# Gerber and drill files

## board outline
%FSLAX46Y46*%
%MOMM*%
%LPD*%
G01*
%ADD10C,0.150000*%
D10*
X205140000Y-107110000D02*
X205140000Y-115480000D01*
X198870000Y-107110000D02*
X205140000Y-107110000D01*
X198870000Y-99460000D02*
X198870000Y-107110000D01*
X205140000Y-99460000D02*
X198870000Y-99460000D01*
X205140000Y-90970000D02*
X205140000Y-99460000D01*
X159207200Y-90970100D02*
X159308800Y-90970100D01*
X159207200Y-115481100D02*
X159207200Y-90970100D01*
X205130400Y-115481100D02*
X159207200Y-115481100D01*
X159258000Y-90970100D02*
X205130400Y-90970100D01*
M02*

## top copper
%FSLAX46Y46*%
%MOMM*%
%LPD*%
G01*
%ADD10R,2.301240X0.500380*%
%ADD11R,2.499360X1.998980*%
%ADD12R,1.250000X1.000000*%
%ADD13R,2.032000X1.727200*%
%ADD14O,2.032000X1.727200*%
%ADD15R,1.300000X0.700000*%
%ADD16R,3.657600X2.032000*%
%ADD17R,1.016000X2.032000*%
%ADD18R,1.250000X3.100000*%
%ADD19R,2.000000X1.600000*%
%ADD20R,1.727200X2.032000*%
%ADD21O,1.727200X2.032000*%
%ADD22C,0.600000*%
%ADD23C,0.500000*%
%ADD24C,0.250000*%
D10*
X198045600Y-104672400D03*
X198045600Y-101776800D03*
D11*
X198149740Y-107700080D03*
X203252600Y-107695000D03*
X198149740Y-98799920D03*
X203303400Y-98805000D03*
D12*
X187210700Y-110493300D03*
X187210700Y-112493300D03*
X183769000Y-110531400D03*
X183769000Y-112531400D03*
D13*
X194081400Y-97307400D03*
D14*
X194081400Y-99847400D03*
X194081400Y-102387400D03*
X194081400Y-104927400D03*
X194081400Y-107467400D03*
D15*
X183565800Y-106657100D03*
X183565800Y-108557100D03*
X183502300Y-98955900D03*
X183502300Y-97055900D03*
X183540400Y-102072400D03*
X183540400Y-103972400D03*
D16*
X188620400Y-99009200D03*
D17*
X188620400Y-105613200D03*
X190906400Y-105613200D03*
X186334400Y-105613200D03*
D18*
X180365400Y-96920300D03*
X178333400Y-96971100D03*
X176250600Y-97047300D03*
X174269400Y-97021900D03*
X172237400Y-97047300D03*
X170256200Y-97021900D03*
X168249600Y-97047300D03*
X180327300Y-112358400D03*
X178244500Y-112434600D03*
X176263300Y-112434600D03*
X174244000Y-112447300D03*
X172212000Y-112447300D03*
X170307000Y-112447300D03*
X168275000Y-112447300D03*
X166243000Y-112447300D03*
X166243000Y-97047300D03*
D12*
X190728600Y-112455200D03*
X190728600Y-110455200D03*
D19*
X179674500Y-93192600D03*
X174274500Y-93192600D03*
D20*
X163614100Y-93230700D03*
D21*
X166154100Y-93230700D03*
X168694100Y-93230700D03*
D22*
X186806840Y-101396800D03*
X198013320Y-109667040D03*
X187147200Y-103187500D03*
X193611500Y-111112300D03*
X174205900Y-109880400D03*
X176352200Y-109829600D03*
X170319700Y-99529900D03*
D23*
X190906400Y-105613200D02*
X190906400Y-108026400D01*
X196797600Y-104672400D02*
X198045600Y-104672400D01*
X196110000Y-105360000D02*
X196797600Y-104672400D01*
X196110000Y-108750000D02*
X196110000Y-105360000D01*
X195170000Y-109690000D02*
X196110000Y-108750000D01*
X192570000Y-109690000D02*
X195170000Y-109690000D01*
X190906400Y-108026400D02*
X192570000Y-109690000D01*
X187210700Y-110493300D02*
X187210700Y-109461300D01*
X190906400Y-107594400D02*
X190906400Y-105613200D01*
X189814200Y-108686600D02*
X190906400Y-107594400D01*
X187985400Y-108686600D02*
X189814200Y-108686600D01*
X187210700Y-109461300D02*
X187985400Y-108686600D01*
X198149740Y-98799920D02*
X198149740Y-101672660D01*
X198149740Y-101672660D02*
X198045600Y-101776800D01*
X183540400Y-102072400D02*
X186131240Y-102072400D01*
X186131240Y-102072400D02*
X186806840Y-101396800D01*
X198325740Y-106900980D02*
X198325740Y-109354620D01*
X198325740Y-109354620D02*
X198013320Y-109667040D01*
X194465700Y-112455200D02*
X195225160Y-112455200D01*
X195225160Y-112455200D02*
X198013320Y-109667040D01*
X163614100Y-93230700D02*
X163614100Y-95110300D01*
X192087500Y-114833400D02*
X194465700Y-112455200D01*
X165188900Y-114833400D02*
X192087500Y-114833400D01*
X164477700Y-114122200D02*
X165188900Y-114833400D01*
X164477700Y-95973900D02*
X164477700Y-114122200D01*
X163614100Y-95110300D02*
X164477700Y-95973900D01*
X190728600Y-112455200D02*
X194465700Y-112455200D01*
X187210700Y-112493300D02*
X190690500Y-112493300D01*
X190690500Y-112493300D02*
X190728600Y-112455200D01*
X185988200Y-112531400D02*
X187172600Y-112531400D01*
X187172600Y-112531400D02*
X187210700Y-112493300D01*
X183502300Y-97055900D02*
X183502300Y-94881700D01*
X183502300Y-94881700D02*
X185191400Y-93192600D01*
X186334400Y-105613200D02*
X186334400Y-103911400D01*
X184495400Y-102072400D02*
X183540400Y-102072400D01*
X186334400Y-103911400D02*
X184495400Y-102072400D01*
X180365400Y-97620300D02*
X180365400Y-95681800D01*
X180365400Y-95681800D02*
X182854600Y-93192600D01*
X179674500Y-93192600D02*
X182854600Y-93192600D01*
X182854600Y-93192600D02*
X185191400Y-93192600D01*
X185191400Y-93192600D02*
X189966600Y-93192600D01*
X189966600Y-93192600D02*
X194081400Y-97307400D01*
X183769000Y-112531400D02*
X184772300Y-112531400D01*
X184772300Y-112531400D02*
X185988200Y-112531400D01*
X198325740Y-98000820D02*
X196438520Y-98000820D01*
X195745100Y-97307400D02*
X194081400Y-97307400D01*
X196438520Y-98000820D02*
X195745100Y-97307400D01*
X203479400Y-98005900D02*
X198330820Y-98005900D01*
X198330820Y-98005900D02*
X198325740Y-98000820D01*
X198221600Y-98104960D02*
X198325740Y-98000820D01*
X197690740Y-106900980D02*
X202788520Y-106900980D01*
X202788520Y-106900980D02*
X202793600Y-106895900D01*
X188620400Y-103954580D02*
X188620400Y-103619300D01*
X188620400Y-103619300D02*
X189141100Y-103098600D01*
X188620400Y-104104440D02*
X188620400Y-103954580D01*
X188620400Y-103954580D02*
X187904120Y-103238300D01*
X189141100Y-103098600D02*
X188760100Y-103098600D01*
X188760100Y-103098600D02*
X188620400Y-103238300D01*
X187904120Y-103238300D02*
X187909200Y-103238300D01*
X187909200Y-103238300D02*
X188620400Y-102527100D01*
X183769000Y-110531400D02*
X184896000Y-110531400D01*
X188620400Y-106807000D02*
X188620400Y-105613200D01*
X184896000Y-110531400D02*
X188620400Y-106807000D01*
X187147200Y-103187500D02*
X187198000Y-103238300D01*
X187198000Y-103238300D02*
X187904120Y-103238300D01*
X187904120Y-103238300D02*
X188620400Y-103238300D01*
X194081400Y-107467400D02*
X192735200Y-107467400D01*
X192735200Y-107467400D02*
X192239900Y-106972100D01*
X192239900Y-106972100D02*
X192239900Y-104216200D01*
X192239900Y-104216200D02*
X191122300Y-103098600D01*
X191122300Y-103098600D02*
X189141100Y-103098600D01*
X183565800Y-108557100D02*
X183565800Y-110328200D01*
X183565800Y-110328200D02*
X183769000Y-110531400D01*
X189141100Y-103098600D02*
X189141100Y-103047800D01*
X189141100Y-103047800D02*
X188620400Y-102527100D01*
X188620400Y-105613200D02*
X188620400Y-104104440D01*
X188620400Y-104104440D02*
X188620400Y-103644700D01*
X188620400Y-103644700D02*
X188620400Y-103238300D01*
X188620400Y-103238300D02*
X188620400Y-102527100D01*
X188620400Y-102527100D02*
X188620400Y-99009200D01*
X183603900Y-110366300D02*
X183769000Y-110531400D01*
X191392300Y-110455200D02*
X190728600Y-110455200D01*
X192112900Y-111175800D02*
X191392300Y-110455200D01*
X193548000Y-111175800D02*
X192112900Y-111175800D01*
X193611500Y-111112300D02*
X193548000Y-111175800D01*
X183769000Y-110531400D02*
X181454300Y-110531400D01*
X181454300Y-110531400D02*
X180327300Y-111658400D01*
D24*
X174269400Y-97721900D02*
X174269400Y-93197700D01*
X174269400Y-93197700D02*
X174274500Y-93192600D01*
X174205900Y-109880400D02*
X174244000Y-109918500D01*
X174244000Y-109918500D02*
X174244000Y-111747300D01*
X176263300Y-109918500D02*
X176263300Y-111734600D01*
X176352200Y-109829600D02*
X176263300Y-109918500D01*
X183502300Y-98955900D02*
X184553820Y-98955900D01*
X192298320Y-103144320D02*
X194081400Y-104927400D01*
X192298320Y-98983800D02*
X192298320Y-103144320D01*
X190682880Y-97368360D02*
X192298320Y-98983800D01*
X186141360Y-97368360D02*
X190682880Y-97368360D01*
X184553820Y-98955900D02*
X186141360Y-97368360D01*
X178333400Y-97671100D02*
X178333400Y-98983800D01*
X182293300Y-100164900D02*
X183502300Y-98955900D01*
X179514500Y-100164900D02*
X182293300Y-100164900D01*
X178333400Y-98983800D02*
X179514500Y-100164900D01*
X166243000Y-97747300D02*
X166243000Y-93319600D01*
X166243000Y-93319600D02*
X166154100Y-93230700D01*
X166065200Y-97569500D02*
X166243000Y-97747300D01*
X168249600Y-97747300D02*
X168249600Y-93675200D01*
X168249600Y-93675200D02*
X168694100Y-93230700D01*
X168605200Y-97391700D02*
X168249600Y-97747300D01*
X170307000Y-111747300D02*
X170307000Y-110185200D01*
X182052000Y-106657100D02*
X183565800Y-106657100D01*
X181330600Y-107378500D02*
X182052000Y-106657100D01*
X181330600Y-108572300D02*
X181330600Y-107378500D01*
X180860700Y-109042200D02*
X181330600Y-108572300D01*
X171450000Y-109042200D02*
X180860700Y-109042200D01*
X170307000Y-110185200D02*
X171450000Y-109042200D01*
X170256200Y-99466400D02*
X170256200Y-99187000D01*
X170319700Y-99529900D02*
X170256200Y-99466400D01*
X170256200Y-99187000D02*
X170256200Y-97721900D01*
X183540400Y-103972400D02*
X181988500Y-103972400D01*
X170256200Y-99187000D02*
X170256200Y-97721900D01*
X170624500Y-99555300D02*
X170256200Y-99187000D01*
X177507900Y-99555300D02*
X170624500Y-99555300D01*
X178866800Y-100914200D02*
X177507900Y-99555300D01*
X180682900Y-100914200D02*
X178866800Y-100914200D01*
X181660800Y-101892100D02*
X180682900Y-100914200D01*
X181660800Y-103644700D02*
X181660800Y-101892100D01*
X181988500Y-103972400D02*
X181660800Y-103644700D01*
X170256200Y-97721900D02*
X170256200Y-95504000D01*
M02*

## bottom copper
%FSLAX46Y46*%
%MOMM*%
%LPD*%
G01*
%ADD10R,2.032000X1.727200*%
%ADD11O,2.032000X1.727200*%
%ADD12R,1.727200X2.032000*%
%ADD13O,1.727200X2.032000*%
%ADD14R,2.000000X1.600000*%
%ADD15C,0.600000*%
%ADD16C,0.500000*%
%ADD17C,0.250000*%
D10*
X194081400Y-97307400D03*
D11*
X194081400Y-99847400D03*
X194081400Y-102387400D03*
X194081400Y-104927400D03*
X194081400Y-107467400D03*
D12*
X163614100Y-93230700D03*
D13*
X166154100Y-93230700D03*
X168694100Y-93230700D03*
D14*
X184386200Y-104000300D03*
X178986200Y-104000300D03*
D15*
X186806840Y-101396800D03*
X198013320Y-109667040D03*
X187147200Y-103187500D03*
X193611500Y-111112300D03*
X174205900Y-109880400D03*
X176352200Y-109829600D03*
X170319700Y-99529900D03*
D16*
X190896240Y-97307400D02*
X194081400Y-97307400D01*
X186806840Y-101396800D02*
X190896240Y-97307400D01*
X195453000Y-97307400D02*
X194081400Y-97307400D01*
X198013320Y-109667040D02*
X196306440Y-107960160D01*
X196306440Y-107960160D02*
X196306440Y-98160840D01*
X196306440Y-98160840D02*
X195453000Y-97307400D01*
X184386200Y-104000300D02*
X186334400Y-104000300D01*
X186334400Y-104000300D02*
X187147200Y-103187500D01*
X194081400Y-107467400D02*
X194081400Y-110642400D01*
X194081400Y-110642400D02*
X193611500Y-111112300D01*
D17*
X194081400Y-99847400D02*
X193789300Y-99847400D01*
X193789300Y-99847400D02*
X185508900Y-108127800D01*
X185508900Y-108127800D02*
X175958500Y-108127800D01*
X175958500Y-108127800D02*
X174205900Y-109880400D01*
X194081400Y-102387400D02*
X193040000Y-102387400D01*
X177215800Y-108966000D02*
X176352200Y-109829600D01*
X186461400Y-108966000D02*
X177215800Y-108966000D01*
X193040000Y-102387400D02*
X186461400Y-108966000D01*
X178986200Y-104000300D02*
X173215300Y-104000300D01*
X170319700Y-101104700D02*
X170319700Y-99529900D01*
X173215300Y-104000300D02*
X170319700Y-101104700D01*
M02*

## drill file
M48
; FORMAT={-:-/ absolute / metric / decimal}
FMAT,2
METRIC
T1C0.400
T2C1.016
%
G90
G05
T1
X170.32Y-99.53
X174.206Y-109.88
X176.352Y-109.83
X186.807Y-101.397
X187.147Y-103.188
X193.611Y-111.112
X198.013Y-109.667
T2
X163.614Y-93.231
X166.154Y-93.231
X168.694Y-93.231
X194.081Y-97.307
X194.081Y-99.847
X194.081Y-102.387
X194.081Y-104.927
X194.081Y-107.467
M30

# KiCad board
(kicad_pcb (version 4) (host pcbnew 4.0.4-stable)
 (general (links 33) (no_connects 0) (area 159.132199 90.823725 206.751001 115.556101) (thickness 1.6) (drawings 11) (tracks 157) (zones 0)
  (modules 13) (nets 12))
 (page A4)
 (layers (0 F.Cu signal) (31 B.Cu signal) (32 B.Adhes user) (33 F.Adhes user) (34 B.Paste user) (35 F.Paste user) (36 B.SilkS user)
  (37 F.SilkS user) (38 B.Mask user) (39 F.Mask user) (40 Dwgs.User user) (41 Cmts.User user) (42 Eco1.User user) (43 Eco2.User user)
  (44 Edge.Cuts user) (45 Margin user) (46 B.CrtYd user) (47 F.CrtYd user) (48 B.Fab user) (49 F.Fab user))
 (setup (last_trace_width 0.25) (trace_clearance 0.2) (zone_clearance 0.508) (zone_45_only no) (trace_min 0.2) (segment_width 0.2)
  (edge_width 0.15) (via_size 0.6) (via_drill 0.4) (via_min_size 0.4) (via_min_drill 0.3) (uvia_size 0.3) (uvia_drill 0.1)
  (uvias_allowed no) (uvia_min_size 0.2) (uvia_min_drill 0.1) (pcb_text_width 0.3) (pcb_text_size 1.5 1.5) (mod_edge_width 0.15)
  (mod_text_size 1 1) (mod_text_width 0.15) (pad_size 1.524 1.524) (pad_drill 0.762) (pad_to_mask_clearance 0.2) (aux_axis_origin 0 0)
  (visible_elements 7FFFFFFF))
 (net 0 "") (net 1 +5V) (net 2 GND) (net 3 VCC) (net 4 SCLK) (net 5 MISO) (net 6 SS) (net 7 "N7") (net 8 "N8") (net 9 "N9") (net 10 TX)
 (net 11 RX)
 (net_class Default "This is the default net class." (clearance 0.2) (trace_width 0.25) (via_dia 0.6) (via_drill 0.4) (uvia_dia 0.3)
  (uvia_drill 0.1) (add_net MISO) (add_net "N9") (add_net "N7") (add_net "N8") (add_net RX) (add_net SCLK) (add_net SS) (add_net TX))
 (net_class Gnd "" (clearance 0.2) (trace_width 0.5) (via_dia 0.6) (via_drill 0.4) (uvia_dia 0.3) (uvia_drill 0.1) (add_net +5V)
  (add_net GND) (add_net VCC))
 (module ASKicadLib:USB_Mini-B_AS (layer F.Cu) (at 201.5 103.25 180)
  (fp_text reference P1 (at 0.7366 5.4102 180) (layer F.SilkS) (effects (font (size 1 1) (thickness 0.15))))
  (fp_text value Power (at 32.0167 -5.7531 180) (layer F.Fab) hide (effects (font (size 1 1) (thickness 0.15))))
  (pad 1 smd rect (at 3.4544 -1.4224 180) (size 2.30124 0.50038) (layers F.Cu F.Paste F.Mask) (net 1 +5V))
  (pad 5 smd rect (at 3.4544 1.4732 180) (size 2.30124 0.50038) (layers F.Cu F.Paste F.Mask) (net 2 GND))
  (pad 6 smd rect (at 3.35026 -4.45008 180) (size 2.49936 1.99898) (layers F.Cu F.Paste F.Mask) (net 2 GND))
  (pad 6 smd rect (at -1.7526 -4.445 180) (size 2.49936 1.99898) (layers F.Cu F.Paste F.Mask) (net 2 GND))
  (pad 6 smd rect (at 3.35026 4.45008 180) (size 2.49936 1.99898) (layers F.Cu F.Paste F.Mask) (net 2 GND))
  (pad 6 smd rect (at -1.8034 4.445 180) (size 2.49936 1.99898) (layers F.Cu F.Paste F.Mask) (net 2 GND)))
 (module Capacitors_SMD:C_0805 (layer F.Cu) (at 187.2107 111.4933 270)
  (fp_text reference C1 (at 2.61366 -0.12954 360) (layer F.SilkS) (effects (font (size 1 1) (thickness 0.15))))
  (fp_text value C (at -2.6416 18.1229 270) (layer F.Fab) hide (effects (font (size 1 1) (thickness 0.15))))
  (pad 1 smd rect (at -1 0 270) (size 1 1.25) (layers F.Cu F.Paste F.Mask) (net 1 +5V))
  (pad 2 smd rect (at 1 0 270) (size 1 1.25) (layers F.Cu F.Paste F.Mask) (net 2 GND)))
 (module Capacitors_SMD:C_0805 (layer F.Cu) (at 183.769 111.5314 270)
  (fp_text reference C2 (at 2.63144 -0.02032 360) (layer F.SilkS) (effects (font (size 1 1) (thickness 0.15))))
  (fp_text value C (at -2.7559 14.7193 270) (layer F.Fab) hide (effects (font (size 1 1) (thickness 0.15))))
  (pad 1 smd rect (at -1 0 270) (size 1 1.25) (layers F.Cu F.Paste F.Mask) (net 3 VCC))
  (pad 2 smd rect (at 1 0 270) (size 1 1.25) (layers F.Cu F.Paste F.Mask) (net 2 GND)))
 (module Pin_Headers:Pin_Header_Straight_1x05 (layer F.Cu) (at 194.0814 97.3074)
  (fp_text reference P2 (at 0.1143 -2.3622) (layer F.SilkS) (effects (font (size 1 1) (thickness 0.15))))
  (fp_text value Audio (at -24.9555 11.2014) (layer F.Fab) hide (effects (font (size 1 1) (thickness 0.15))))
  (pad 1 thru_hole rect (at 0 0) (size 2.032 1.7272) (drill 1.016) (layers *.Cu *.Mask) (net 2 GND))
  (pad 2 thru_hole oval (at 0 2.54) (size 2.032 1.7272) (drill 1.016) (layers *.Cu *.Mask) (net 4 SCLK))
  (pad 3 thru_hole oval (at 0 5.08) (size 2.032 1.7272) (drill 1.016) (layers *.Cu *.Mask) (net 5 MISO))
  (pad 4 thru_hole oval (at 0 7.62) (size 2.032 1.7272) (drill 1.016) (layers *.Cu *.Mask) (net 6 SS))
  (pad 5 thru_hole oval (at 0 10.16) (size 2.032 1.7272) (drill 1.016) (layers *.Cu *.Mask) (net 3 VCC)))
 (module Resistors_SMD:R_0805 (layer F.Cu) (at 183.5658 107.6071 270)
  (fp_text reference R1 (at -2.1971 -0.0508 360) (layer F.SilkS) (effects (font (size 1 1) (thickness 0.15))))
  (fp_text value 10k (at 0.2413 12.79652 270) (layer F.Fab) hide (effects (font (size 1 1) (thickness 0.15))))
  (pad 1 smd rect (at -0.95 0 270) (size 0.7 1.3) (layers F.Cu F.Paste F.Mask) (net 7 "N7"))
  (pad 2 smd rect (at 0.95 0 270) (size 0.7 1.3) (layers F.Cu F.Paste F.Mask) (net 3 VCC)))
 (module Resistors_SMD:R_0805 (layer F.Cu) (at 183.5023 98.0059 90)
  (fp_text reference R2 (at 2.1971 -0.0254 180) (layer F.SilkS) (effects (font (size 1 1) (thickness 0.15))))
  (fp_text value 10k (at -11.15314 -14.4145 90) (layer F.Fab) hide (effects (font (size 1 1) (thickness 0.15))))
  (pad 1 smd rect (at -0.95 0 90) (size 0.7 1.3) (layers F.Cu F.Paste F.Mask) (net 6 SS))
  (pad 2 smd rect (at 0.95 0 90) (size 0.7 1.3) (layers F.Cu F.Paste F.Mask) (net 2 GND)))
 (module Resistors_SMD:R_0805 (layer F.Cu) (at 183.5404 103.0224 270)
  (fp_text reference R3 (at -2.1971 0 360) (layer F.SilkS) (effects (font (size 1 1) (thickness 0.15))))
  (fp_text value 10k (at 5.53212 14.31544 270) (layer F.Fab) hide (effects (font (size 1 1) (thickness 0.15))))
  (pad 1 smd rect (at -0.95 0 270) (size 0.7 1.3) (layers F.Cu F.Paste F.Mask) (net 2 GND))
  (pad 2 smd rect (at 0.95 0 270) (size 0.7 1.3) (layers F.Cu F.Paste F.Mask) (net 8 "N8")))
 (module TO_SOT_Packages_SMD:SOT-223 (layer F.Cu) (at 188.6204 102.3112)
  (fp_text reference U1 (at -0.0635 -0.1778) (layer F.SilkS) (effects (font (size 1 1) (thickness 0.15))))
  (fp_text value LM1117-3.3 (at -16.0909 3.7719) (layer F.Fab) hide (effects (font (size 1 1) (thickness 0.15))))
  (pad 4 smd rect (at 0 -3.302) (size 3.6576 2.032) (layers F.Cu F.Paste F.Mask) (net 3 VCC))
  (pad 2 smd rect (at 0 3.302) (size 1.016 2.032) (layers F.Cu F.Paste F.Mask) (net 3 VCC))
  (pad 3 smd rect (at 2.286 3.302) (size 1.016 2.032) (layers F.Cu F.Paste F.Mask) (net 1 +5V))
  (pad 1 smd rect (at -2.286 3.302) (size 1.016 2.032) (layers F.Cu F.Paste F.Mask) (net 2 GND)))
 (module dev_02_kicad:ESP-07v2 (layer F.Cu) (at 166.243 111.7473 90)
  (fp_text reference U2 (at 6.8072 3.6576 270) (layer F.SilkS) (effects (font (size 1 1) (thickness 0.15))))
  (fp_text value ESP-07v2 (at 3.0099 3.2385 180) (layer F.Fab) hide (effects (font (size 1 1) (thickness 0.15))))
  (pad 9 smd rect (at 14.127 14.1224 90) (size 3.1 1.25) (drill (offset 0.7 0)) (layers F.Cu F.Paste F.Mask) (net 2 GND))
  (pad 10 smd rect (at 14.0762 12.0904 90) (size 3.1 1.25) (drill (offset 0.7 0)) (layers F.Cu F.Paste F.Mask) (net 6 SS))
  (pad 11 smd rect (at 14 10.0076 90) (size 3.1 1.25) (drill (offset 0.7 0)) (layers F.Cu F.Paste F.Mask))
  (pad 12 smd rect (at 14.0254 8.0264 90) (size 3.1 1.25) (drill (offset 0.7 0)) (layers F.Cu F.Paste F.Mask) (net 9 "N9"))
  (pad 13 smd rect (at 14 5.9944 90) (size 3.1 1.25) (drill (offset 0.7 0)) (layers F.Cu F.Paste F.Mask))
  (pad 14 smd rect (at 14.0254 4.0132 90) (size 3.1 1.25) (drill (offset 0.7 0)) (layers F.Cu F.Paste F.Mask) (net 8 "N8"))
  (pad 15 smd rect (at 14 2.0066 90) (size 3.1 1.25) (drill (offset 0.7 0)) (layers F.Cu F.Paste F.Mask) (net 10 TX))
  (pad 8 smd rect (at 0.0889 14.0843 90) (size 3.1 1.25) (drill (offset -0.7 0)) (layers F.Cu F.Paste F.Mask) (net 3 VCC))
  (pad 7 smd rect (at 0.0127 12.0015 90) (size 3.1 1.25) (drill (offset -0.7 0)) (layers F.Cu F.Paste F.Mask))
  (pad 6 smd rect (at 0.0127 10.0203 90) (size 3.1 1.25) (drill (offset -0.7 0)) (layers F.Cu F.Paste F.Mask) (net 5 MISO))
  (pad 5 smd rect (at 0 8.001 90) (size 3.1 1.25) (drill (offset -0.7 0)) (layers F.Cu F.Paste F.Mask) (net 4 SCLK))
  (pad 4 smd rect (at 0 5.969 90) (size 3.1 1.25) (drill (offset -0.7 0)) (layers F.Cu F.Paste F.Mask))
  (pad 3 smd rect (at 0 4.064 90) (size 3.1 1.25) (drill (offset -0.7 0)) (layers F.Cu F.Paste F.Mask) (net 7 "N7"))
  (pad 2 smd rect (at 0 2.032 90) (size 3.1 1.25) (drill (offset -0.7 0)) (layers F.Cu F.Paste F.Mask))
  (pad 1 smd rect (at 0 0 90) (size 3.1 1.25) (drill (offset -0.7 0)) (layers F.Cu F.Paste F.Mask))
  (pad 16 smd rect (at 14 0 90) (size 3.1 1.25) (drill (offset 0.7 0)) (layers F.Cu F.Paste F.Mask) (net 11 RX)))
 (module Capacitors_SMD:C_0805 (layer F.Cu) (at 190.7286 111.4552 90)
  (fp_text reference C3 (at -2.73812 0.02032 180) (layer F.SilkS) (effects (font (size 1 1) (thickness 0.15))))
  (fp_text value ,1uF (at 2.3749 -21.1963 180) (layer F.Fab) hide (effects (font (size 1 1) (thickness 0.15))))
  (pad 1 smd rect (at -1 0 90) (size 1 1.25) (layers F.Cu F.Paste F.Mask) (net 2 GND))
  (pad 2 smd rect (at 1 0 90) (size 1 1.25) (layers F.Cu F.Paste F.Mask) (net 3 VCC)))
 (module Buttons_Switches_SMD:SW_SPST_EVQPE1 (layer F.Cu) (at 176.9745 93.1926)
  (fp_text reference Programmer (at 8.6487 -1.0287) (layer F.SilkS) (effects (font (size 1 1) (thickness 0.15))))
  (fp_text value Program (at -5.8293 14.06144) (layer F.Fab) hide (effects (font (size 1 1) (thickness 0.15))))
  (pad 2 smd rect (at 2.7 0) (size 2 1.6) (layers F.Cu F.Paste F.Mask) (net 2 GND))
  (pad 1 smd rect (at -2.7 0) (size 2 1.6) (layers F.Cu F.Paste F.Mask) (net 9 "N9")))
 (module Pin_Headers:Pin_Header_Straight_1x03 (layer F.Cu) (at 163.6141 93.2307 90)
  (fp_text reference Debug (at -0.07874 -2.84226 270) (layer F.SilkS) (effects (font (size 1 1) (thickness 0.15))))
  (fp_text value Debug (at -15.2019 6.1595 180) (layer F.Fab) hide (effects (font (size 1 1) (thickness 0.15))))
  (pad 1 thru_hole rect (at 0 0 90) (size 2.032 1.7272) (drill 1.016) (layers *.Cu *.Mask) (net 2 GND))
  (pad 2 thru_hole oval (at 0 2.54 90) (size 2.032 1.7272) (drill 1.016) (layers *.Cu *.Mask) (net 11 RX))
  (pad 3 thru_hole oval (at 0 5.08 90) (size 2.032 1.7272) (drill 1.016) (layers *.Cu *.Mask) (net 10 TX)))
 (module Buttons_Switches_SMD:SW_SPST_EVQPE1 (layer B.Cu) (at 181.6862 104.0003)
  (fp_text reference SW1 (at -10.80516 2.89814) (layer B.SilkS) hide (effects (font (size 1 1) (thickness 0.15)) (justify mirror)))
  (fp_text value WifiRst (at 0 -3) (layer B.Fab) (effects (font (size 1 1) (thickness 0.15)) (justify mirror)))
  (pad 2 smd rect (at 2.7 0) (size 2 1.6) (layers B.Cu B.Paste B.Mask) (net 3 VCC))
  (pad 1 smd rect (at -2.7 0) (size 2 1.6) (layers B.Cu B.Paste B.Mask) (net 8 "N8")))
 (gr_line (start 205.14 107.11) (end 205.14 115.48) (angle 90) (layer Edge.Cuts) (width 0.15))
 (gr_line (start 198.87 107.11) (end 205.14 107.11) (angle 90) (layer Edge.Cuts) (width 0.15))
 (gr_line (start 198.87 99.46) (end 198.87 107.11) (angle 90) (layer Edge.Cuts) (width 0.15))
 (gr_line (start 205.14 99.46) (end 198.87 99.46) (angle 90) (layer Edge.Cuts) (width 0.15))
 (gr_line (start 205.14 90.97) (end 205.14 99.46) (angle 90) (layer Edge.Cuts) (width 0.15))
 (gr_line (start 159.2072 90.9701) (end 159.3088 90.9701) (angle 90) (layer Edge.Cuts) (width 0.15))
 (gr_line (start 159.2072 115.4811) (end 159.2072 90.9701) (angle 90) (layer Edge.Cuts) (width 0.15))
 (gr_line (start 205.1304 115.4811) (end 159.2072 115.4811) (angle 90) (layer Edge.Cuts) (width 0.15))
 (gr_line (start 159.258 90.9701) (end 205.1304 90.9701) (angle 90) (layer Edge.Cuts) (width 0.15))
 (segment (start 190.9064 105.6132) (end 190.9064 108.0264) (width 0.5) (layer F.Cu) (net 1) (status 400000))
 (segment (start 196.7976 104.6724) (end 198.0456 104.6724) (width 0.5) (layer F.Cu) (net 1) (status 800000))
 (segment (start 196.11 105.36) (end 196.7976 104.6724) (width 0.5) (layer F.Cu) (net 1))
 (segment (start 196.11 108.75) (end 196.11 105.36) (width 0.5) (layer F.Cu) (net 1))
 (segment (start 195.17 109.69) (end 196.11 108.75) (width 0.5) (layer F.Cu) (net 1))
 (segment (start 192.57 109.69) (end 195.17 109.69) (width 0.5) (layer F.Cu) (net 1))
 (segment (start 190.9064 108.0264) (end 192.57 109.69) (width 0.5) (layer F.Cu) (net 1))
 (segment (start 187.2107 110.4933) (end 187.2107 109.4613) (width 0.5) (layer F.Cu) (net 1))
 (segment (start 190.9064 107.5944) (end 190.9064 105.6132) (width 0.5) (layer F.Cu) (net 1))
 (segment (start 189.8142 108.6866) (end 190.9064 107.5944) (width 0.5) (layer F.Cu) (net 1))
 (segment (start 187.9854 108.6866) (end 189.8142 108.6866) (width 0.5) (layer F.Cu) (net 1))
 (segment (start 187.2107 109.4613) (end 187.9854 108.6866) (width 0.5) (layer F.Cu) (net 1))
 (segment (start 198.14974 98.79992) (end 198.14974 101.67266) (width 0.5) (layer F.Cu) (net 2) (status C00000))
 (segment (start 198.14974 101.67266) (end 198.0456 101.7768) (width 0.5) (layer F.Cu) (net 2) (status C00000))
 (segment (start 183.5404 102.0724) (end 186.13124 102.0724) (width 0.5) (layer F.Cu) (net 2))
 (segment (start 190.89624 97.3074) (end 194.0814 97.3074) (width 0.5) (layer B.Cu) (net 2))
 (segment (start 186.80684 101.3968) (end 190.89624 97.3074) (width 0.5) (layer B.Cu) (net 2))
 (via (at 186.80684 101.3968) (size 0.6) (drill 0.4) (layers F.Cu B.Cu) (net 2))
 (segment (start 186.13124 102.0724) (end 186.80684 101.3968) (width 0.5) (layer F.Cu) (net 2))
 (segment (start 198.32574 106.90098) (end 198.32574 109.35462) (width 0.5) (layer F.Cu) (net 2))
 (segment (start 198.32574 109.35462) (end 198.01332 109.66704) (width 0.5) (layer F.Cu) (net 2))
 (segment (start 194.4657 112.4552) (end 195.22516 112.4552) (width 0.5) (layer F.Cu) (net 2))
 (segment (start 195.453 97.3074) (end 194.0814 97.3074) (width 0.5) (layer B.Cu) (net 2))
 (via (at 198.01332 109.66704) (size 0.6) (drill 0.4) (layers F.Cu B.Cu) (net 2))
 (segment (start 198.01332 109.66704) (end 196.30644 107.96016) (width 0.5) (layer B.Cu) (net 2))
 (segment (start 196.30644 107.96016) (end 196.30644 98.16084) (width 0.5) (layer B.Cu) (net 2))
 (segment (start 196.30644 98.16084) (end 195.453 97.3074) (width 0.5) (layer B.Cu) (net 2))
 (segment (start 195.22516 112.4552) (end 198.01332 109.66704) (width 0.5) (layer F.Cu) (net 2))
 (segment (start 163.6141 93.2307) (end 163.6141 95.1103) (width 0.5) (layer F.Cu) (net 2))
 (segment (start 192.0875 114.8334) (end 194.4657 112.4552) (width 0.5) (layer F.Cu) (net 2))
 (segment (start 165.1889 114.8334) (end 192.0875 114.8334) (width 0.5) (layer F.Cu) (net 2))
 (segment (start 164.4777 114.1222) (end 165.1889 114.8334) (width 0.5) (layer F.Cu) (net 2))
 (segment (start 164.4777 95.9739) (end 164.4777 114.1222) (width 0.5) (layer F.Cu) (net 2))
 (segment (start 163.6141 95.1103) (end 164.4777 95.9739) (width 0.5) (layer F.Cu) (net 2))
 (segment (start 190.7286 112.4552) (end 194.4657 112.4552) (width 0.5) (layer F.Cu) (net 2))
 (segment (start 187.2107 112.4933) (end 190.6905 112.4933) (width 0.5) (layer F.Cu) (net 2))
 (segment (start 190.6905 112.4933) (end 190.7286 112.4552) (width 0.5) (layer F.Cu) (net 2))
 (segment (start 185.9882 112.5314) (end 187.1726 112.5314) (width 0.5) (layer F.Cu) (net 2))
 (segment (start 187.1726 112.5314) (end 187.2107 112.4933) (width 0.5) (layer F.Cu) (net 2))
 (segment (start 183.5023 97.0559) (end 183.5023 94.8817) (width 0.5) (layer F.Cu) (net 2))
 (segment (start 183.5023 94.8817) (end 185.1914 93.1926) (width 0.5) (layer F.Cu) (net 2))
 (segment (start 186.3344 105.6132) (end 186.3344 103.9114) (width 0.5) (layer F.Cu) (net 2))
 (segment (start 184.4954 102.0724) (end 183.5404 102.0724) (width 0.5) (layer F.Cu) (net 2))
 (segment (start 186.3344 103.9114) (end 184.4954 102.0724) (width 0.5) (layer F.Cu) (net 2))
 (segment (start 180.3654 97.6203) (end 180.3654 95.6818) (width 0.5) (layer F.Cu) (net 2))
 (segment (start 180.3654 95.6818) (end 182.8546 93.1926) (width 0.5) (layer F.Cu) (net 2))
 (segment (start 179.6745 93.1926) (end 182.8546 93.1926) (width 0.5) (layer F.Cu) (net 2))
 (segment (start 182.8546 93.1926) (end 185.1914 93.1926) (width 0.5) (layer F.Cu) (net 2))
 (segment (start 185.1914 93.1926) (end 189.9666 93.1926) (width 0.5) (layer F.Cu) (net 2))
 (segment (start 189.9666 93.1926) (end 194.0814 97.3074) (width 0.5) (layer F.Cu) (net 2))
 (segment (start 183.769 112.5314) (end 184.7723 112.5314) (width 0.5) (layer F.Cu) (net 2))
 (segment (start 184.7723 112.5314) (end 185.9882 112.5314) (width 0.5) (layer F.Cu) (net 2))
 (segment (start 198.32574 98.00082) (end 196.43852 98.00082) (width 0.5) (layer F.Cu) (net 2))
 (segment (start 195.7451 97.3074) (end 194.0814 97.3074) (width 0.5) (layer F.Cu) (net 2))
 (segment (start 196.43852 98.00082) (end 195.7451 97.3074) (width 0.5) (layer F.Cu) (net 2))
 (segment (start 203.4794 98.0059) (end 198.33082 98.0059) (width 0.5) (layer F.Cu) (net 2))
 (segment (start 198.33082 98.0059) (end 198.32574 98.00082) (width 0.5) (layer F.Cu) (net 2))
 (segment (start 198.2216 98.10496) (end 198.32574 98.00082) (width 0.5) (layer F.Cu) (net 2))
 (segment (start 197.69074 106.90098) (end 202.78852 106.90098) (width 0.5) (layer F.Cu) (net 2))
 (segment (start 202.78852 106.90098) (end 202.7936 106.8959) (width 0.5) (layer F.Cu) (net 2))
 (segment (start 188.6204 103.95458) (end 188.6204 103.6193) (width 0.5) (layer F.Cu) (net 3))
 (segment (start 188.6204 103.6193) (end 189.1411 103.0986) (width 0.5) (layer F.Cu) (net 3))
 (segment (start 188.6204 104.10444) (end 188.6204 103.95458) (width 0.5) (layer F.Cu) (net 3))
 (segment (start 188.6204 103.95458) (end 187.90412 103.2383) (width 0.5) (layer F.Cu) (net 3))
 (segment (start 189.1411 103.0986) (end 188.7601 103.0986) (width 0.5) (layer F.Cu) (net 3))
 (segment (start 188.7601 103.0986) (end 188.6204 103.2383) (width 0.5) (layer F.Cu) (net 3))
 (segment (start 187.90412 103.2383) (end 187.9092 103.2383) (width 0.5) (layer F.Cu) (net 3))
 (segment (start 187.9092 103.2383) (end 188.6204 102.5271) (width 0.5) (layer F.Cu) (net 3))
 (segment (start 183.769 110.5314) (end 184.896 110.5314) (width 0.5) (layer F.Cu) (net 3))
 (segment (start 188.6204 106.807) (end 188.6204 105.6132) (width 0.5) (layer F.Cu) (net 3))
 (segment (start 184.896 110.5314) (end 188.6204 106.807) (width 0.5) (layer F.Cu) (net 3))
 (segment (start 184.3862 104.0003) (end 186.3344 104.0003) (width 0.5) (layer B.Cu) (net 3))
 (segment (start 186.3344 104.0003) (end 187.1472 103.1875) (width 0.5) (layer B.Cu) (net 3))
 (via (at 187.1472 103.1875) (size 0.6) (drill 0.4) (layers F.Cu B.Cu) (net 3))
 (segment (start 187.1472 103.1875) (end 187.198 103.2383) (width 0.5) (layer F.Cu) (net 3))
 (segment (start 187.198 103.2383) (end 187.90412 103.2383) (width 0.5) (layer F.Cu) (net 3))
 (segment (start 187.90412 103.2383) (end 188.6204 103.2383) (width 0.5) (layer F.Cu) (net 3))
 (segment (start 194.0814 107.4674) (end 192.7352 107.4674) (width 0.5) (layer F.Cu) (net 3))
 (segment (start 192.7352 107.4674) (end 192.2399 106.9721) (width 0.5) (layer F.Cu) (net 3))
 (segment (start 192.2399 106.9721) (end 192.2399 104.2162) (width 0.5) (layer F.Cu) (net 3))
 (segment (start 192.2399 104.2162) (end 191.1223 103.0986) (width 0.5) (layer F.Cu) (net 3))
 (segment (start 191.1223 103.0986) (end 189.1411 103.0986) (width 0.5) (layer F.Cu) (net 3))
 (segment (start 183.5658 108.5571) (end 183.5658 110.3282) (width 0.5) (layer F.Cu) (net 3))
 (segment (start 183.5658 110.3282) (end 183.769 110.5314) (width 0.5) (layer F.Cu) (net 3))
 (segment (start 189.1411 103.0986) (end 189.1411 103.0478) (width 0.5) (layer F.Cu) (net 3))
 (segment (start 189.1411 103.0478) (end 188.6204 102.5271) (width 0.5) (layer F.Cu) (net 3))
 (segment (start 188.6204 105.6132) (end 188.6204 104.10444) (width 0.5) (layer F.Cu) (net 3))
 (segment (start 188.6204 104.10444) (end 188.6204 103.6447) (width 0.5) (layer F.Cu) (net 3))
 (segment (start 188.6204 103.6447) (end 188.6204 103.2383) (width 0.5) (layer F.Cu) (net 3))
 (segment (start 188.6204 103.2383) (end 188.6204 102.5271) (width 0.5) (layer F.Cu) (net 3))
 (segment (start 188.6204 102.5271) (end 188.6204 99.0092) (width 0.5) (layer F.Cu) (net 3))
 (segment (start 183.6039 110.3663) (end 183.769 110.5314) (width 0.5) (layer F.Cu) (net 3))
 (segment (start 194.0814 107.4674) (end 194.0814 110.6424) (width 0.5) (layer B.Cu) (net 3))
 (segment (start 191.3923 110.4552) (end 190.7286 110.4552) (width 0.5) (layer F.Cu) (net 3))
 (segment (start 192.1129 111.1758) (end 191.3923 110.4552) (width 0.5) (layer F.Cu) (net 3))
 (segment (start 193.548 111.1758) (end 192.1129 111.1758) (width 0.5) (layer F.Cu) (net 3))
 (segment (start 193.6115 111.1123) (end 193.548 111.1758) (width 0.5) (layer F.Cu) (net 3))
 (via (at 193.6115 111.1123) (size 0.6) (drill 0.4) (layers F.Cu B.Cu) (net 3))
 (segment (start 194.0814 110.6424) (end 193.6115 111.1123) (width 0.5) (layer B.Cu) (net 3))
 (segment (start 183.769 110.5314) (end 181.4543 110.5314) (width 0.5) (layer F.Cu) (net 3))
 (segment (start 181.4543 110.5314) (end 180.3273 111.6584) (width 0.5) (layer F.Cu) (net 3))
 (segment (start 174.2694 97.7219) (end 174.2694 93.1977) (width 0.25) (layer F.Cu) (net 9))
 (segment (start 174.2694 93.1977) (end 174.2745 93.1926) (width 0.25) (layer F.Cu) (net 9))
 (segment (start 194.0814 99.8474) (end 193.7893 99.8474) (width 0.25) (layer B.Cu) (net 4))
 (segment (start 193.7893 99.8474) (end 185.5089 108.1278) (width 0.25) (layer B.Cu) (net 4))
 (segment (start 185.5089 108.1278) (end 175.9585 108.1278) (width 0.25) (layer B.Cu) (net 4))
 (segment (start 175.9585 108.1278) (end 174.2059 109.8804) (width 0.25) (layer B.Cu) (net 4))
 (via (at 174.2059 109.8804) (size 0.6) (drill 0.4) (layers F.Cu B.Cu) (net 4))
 (segment (start 174.2059 109.8804) (end 174.244 109.9185) (width 0.25) (layer F.Cu) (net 4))
 (segment (start 174.244 109.9185) (end 174.244 111.7473) (width 0.25) (layer F.Cu) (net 4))
 (segment (start 194.0814 102.3874) (end 193.04 102.3874) (width 0.25) (layer B.Cu) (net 5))
 (segment (start 176.2633 109.9185) (end 176.2633 111.7346) (width 0.25) (layer F.Cu) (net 5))
 (segment (start 176.3522 109.8296) (end 176.2633 109.9185) (width 0.25) (layer F.Cu) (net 5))
 (via (at 176.3522 109.8296) (size 0.6) (drill 0.4) (layers F.Cu B.Cu) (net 5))
 (segment (start 177.2158 108.966) (end 176.3522 109.8296) (width 0.25) (layer B.Cu) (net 5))
 (segment (start 186.4614 108.966) (end 177.2158 108.966) (width 0.25) (layer B.Cu) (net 5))
 (segment (start 193.04 102.3874) (end 186.4614 108.966) (width 0.25) (layer B.Cu) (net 5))
 (segment (start 183.5023 98.9559) (end 184.55382 98.9559) (width 0.25) (layer F.Cu) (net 6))
 (segment (start 192.29832 103.14432) (end 194.0814 104.9274) (width 0.25) (layer F.Cu) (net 6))
 (segment (start 192.29832 98.9838) (end 192.29832 103.14432) (width 0.25) (layer F.Cu) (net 6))
 (segment (start 190.68288 97.36836) (end 192.29832 98.9838) (width 0.25) (layer F.Cu) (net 6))
 (segment (start 186.14136 97.36836) (end 190.68288 97.36836) (width 0.25) (layer F.Cu) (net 6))
 (segment (start 184.55382 98.9559) (end 186.14136 97.36836) (width 0.25) (layer F.Cu) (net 6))
 (segment (start 178.3334 97.6711) (end 178.3334 98.9838) (width 0.25) (layer F.Cu) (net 6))
 (segment (start 182.2933 100.1649) (end 183.5023 98.9559) (width 0.25) (layer F.Cu) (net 6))
 (segment (start 179.5145 100.1649) (end 182.2933 100.1649) (width 0.25) (layer F.Cu) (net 6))
 (segment (start 178.3334 98.9838) (end 179.5145 100.1649) (width 0.25) (layer F.Cu) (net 6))
 (segment (start 166.243 97.7473) (end 166.243 93.3196) (width 0.25) (layer F.Cu) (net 11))
 (segment (start 166.243 93.3196) (end 166.1541 93.2307) (width 0.25) (layer F.Cu) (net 11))
 (segment (start 166.0652 97.5695) (end 166.243 97.7473) (width 0.25) (layer F.Cu) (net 11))
 (segment (start 168.2496 97.7473) (end 168.2496 93.6752) (width 0.25) (layer F.Cu) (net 10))
 (segment (start 168.2496 93.6752) (end 168.6941 93.2307) (width 0.25) (layer F.Cu) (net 10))
 (segment (start 168.6052 97.3917) (end 168.2496 97.7473) (width 0.25) (layer F.Cu) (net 10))
 (segment (start 170.307 111.7473) (end 170.307 110.1852) (width 0.25) (layer F.Cu) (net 7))
 (segment (start 182.052 106.6571) (end 183.5658 106.6571) (width 0.25) (layer F.Cu) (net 7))
 (segment (start 181.3306 107.3785) (end 182.052 106.6571) (width 0.25) (layer F.Cu) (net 7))
 (segment (start 181.3306 108.5723) (end 181.3306 107.3785) (width 0.25) (layer F.Cu) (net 7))
 (segment (start 180.8607 109.0422) (end 181.3306 108.5723) (width 0.25) (layer F.Cu) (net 7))
 (segment (start 171.45 109.0422) (end 180.8607 109.0422) (width 0.25) (layer F.Cu) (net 7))
 (segment (start 170.307 110.1852) (end 171.45 109.0422) (width 0.25) (layer F.Cu) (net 7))
 (segment (start 178.9862 104.0003) (end 173.2153 104.0003) (width 0.25) (layer B.Cu) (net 8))
 (segment (start 170.2562 99.4664) (end 170.2562 99.187) (width 0.25) (layer F.Cu) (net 8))
 (segment (start 170.3197 99.5299) (end 170.2562 99.4664) (width 0.25) (layer F.Cu) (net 8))
 (via (at 170.3197 99.5299) (size 0.6) (drill 0.4) (layers F.Cu B.Cu) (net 8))
 (segment (start 170.3197 101.1047) (end 170.3197 99.5299) (width 0.25) (layer B.Cu) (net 8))
 (segment (start 173.2153 104.0003) (end 170.3197 101.1047) (width 0.25) (layer B.Cu) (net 8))
 (segment (start 170.2562 99.187) (end 170.2562 97.7219) (width 0.25) (layer F.Cu) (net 8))
 (segment (start 183.5404 103.9724) (end 181.9885 103.9724) (width 0.25) (layer F.Cu) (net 8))
 (segment (start 170.2562 99.187) (end 170.2562 97.7219) (width 0.25) (layer F.Cu) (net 8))
 (segment (start 170.6245 99.5553) (end 170.2562 99.187) (width 0.25) (layer F.Cu) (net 8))
 (segment (start 177.5079 99.5553) (end 170.6245 99.5553) (width 0.25) (layer F.Cu) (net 8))
 (segment (start 178.8668 100.9142) (end 177.5079 99.5553) (width 0.25) (layer F.Cu) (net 8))
 (segment (start 180.6829 100.9142) (end 178.8668 100.9142) (width 0.25) (layer F.Cu) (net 8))
 (segment (start 181.6608 101.8921) (end 180.6829 100.9142) (width 0.25) (layer F.Cu) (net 8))
 (segment (start 181.6608 103.6447) (end 181.6608 101.8921) (width 0.25) (layer F.Cu) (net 8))
 (segment (start 181.9885 103.9724) (end 181.6608 103.6447) (width 0.25) (layer F.Cu) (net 8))
 (segment (start 170.2562 97.7219) (end 170.2562 95.504) (width 0.25) (layer F.Cu) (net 8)))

